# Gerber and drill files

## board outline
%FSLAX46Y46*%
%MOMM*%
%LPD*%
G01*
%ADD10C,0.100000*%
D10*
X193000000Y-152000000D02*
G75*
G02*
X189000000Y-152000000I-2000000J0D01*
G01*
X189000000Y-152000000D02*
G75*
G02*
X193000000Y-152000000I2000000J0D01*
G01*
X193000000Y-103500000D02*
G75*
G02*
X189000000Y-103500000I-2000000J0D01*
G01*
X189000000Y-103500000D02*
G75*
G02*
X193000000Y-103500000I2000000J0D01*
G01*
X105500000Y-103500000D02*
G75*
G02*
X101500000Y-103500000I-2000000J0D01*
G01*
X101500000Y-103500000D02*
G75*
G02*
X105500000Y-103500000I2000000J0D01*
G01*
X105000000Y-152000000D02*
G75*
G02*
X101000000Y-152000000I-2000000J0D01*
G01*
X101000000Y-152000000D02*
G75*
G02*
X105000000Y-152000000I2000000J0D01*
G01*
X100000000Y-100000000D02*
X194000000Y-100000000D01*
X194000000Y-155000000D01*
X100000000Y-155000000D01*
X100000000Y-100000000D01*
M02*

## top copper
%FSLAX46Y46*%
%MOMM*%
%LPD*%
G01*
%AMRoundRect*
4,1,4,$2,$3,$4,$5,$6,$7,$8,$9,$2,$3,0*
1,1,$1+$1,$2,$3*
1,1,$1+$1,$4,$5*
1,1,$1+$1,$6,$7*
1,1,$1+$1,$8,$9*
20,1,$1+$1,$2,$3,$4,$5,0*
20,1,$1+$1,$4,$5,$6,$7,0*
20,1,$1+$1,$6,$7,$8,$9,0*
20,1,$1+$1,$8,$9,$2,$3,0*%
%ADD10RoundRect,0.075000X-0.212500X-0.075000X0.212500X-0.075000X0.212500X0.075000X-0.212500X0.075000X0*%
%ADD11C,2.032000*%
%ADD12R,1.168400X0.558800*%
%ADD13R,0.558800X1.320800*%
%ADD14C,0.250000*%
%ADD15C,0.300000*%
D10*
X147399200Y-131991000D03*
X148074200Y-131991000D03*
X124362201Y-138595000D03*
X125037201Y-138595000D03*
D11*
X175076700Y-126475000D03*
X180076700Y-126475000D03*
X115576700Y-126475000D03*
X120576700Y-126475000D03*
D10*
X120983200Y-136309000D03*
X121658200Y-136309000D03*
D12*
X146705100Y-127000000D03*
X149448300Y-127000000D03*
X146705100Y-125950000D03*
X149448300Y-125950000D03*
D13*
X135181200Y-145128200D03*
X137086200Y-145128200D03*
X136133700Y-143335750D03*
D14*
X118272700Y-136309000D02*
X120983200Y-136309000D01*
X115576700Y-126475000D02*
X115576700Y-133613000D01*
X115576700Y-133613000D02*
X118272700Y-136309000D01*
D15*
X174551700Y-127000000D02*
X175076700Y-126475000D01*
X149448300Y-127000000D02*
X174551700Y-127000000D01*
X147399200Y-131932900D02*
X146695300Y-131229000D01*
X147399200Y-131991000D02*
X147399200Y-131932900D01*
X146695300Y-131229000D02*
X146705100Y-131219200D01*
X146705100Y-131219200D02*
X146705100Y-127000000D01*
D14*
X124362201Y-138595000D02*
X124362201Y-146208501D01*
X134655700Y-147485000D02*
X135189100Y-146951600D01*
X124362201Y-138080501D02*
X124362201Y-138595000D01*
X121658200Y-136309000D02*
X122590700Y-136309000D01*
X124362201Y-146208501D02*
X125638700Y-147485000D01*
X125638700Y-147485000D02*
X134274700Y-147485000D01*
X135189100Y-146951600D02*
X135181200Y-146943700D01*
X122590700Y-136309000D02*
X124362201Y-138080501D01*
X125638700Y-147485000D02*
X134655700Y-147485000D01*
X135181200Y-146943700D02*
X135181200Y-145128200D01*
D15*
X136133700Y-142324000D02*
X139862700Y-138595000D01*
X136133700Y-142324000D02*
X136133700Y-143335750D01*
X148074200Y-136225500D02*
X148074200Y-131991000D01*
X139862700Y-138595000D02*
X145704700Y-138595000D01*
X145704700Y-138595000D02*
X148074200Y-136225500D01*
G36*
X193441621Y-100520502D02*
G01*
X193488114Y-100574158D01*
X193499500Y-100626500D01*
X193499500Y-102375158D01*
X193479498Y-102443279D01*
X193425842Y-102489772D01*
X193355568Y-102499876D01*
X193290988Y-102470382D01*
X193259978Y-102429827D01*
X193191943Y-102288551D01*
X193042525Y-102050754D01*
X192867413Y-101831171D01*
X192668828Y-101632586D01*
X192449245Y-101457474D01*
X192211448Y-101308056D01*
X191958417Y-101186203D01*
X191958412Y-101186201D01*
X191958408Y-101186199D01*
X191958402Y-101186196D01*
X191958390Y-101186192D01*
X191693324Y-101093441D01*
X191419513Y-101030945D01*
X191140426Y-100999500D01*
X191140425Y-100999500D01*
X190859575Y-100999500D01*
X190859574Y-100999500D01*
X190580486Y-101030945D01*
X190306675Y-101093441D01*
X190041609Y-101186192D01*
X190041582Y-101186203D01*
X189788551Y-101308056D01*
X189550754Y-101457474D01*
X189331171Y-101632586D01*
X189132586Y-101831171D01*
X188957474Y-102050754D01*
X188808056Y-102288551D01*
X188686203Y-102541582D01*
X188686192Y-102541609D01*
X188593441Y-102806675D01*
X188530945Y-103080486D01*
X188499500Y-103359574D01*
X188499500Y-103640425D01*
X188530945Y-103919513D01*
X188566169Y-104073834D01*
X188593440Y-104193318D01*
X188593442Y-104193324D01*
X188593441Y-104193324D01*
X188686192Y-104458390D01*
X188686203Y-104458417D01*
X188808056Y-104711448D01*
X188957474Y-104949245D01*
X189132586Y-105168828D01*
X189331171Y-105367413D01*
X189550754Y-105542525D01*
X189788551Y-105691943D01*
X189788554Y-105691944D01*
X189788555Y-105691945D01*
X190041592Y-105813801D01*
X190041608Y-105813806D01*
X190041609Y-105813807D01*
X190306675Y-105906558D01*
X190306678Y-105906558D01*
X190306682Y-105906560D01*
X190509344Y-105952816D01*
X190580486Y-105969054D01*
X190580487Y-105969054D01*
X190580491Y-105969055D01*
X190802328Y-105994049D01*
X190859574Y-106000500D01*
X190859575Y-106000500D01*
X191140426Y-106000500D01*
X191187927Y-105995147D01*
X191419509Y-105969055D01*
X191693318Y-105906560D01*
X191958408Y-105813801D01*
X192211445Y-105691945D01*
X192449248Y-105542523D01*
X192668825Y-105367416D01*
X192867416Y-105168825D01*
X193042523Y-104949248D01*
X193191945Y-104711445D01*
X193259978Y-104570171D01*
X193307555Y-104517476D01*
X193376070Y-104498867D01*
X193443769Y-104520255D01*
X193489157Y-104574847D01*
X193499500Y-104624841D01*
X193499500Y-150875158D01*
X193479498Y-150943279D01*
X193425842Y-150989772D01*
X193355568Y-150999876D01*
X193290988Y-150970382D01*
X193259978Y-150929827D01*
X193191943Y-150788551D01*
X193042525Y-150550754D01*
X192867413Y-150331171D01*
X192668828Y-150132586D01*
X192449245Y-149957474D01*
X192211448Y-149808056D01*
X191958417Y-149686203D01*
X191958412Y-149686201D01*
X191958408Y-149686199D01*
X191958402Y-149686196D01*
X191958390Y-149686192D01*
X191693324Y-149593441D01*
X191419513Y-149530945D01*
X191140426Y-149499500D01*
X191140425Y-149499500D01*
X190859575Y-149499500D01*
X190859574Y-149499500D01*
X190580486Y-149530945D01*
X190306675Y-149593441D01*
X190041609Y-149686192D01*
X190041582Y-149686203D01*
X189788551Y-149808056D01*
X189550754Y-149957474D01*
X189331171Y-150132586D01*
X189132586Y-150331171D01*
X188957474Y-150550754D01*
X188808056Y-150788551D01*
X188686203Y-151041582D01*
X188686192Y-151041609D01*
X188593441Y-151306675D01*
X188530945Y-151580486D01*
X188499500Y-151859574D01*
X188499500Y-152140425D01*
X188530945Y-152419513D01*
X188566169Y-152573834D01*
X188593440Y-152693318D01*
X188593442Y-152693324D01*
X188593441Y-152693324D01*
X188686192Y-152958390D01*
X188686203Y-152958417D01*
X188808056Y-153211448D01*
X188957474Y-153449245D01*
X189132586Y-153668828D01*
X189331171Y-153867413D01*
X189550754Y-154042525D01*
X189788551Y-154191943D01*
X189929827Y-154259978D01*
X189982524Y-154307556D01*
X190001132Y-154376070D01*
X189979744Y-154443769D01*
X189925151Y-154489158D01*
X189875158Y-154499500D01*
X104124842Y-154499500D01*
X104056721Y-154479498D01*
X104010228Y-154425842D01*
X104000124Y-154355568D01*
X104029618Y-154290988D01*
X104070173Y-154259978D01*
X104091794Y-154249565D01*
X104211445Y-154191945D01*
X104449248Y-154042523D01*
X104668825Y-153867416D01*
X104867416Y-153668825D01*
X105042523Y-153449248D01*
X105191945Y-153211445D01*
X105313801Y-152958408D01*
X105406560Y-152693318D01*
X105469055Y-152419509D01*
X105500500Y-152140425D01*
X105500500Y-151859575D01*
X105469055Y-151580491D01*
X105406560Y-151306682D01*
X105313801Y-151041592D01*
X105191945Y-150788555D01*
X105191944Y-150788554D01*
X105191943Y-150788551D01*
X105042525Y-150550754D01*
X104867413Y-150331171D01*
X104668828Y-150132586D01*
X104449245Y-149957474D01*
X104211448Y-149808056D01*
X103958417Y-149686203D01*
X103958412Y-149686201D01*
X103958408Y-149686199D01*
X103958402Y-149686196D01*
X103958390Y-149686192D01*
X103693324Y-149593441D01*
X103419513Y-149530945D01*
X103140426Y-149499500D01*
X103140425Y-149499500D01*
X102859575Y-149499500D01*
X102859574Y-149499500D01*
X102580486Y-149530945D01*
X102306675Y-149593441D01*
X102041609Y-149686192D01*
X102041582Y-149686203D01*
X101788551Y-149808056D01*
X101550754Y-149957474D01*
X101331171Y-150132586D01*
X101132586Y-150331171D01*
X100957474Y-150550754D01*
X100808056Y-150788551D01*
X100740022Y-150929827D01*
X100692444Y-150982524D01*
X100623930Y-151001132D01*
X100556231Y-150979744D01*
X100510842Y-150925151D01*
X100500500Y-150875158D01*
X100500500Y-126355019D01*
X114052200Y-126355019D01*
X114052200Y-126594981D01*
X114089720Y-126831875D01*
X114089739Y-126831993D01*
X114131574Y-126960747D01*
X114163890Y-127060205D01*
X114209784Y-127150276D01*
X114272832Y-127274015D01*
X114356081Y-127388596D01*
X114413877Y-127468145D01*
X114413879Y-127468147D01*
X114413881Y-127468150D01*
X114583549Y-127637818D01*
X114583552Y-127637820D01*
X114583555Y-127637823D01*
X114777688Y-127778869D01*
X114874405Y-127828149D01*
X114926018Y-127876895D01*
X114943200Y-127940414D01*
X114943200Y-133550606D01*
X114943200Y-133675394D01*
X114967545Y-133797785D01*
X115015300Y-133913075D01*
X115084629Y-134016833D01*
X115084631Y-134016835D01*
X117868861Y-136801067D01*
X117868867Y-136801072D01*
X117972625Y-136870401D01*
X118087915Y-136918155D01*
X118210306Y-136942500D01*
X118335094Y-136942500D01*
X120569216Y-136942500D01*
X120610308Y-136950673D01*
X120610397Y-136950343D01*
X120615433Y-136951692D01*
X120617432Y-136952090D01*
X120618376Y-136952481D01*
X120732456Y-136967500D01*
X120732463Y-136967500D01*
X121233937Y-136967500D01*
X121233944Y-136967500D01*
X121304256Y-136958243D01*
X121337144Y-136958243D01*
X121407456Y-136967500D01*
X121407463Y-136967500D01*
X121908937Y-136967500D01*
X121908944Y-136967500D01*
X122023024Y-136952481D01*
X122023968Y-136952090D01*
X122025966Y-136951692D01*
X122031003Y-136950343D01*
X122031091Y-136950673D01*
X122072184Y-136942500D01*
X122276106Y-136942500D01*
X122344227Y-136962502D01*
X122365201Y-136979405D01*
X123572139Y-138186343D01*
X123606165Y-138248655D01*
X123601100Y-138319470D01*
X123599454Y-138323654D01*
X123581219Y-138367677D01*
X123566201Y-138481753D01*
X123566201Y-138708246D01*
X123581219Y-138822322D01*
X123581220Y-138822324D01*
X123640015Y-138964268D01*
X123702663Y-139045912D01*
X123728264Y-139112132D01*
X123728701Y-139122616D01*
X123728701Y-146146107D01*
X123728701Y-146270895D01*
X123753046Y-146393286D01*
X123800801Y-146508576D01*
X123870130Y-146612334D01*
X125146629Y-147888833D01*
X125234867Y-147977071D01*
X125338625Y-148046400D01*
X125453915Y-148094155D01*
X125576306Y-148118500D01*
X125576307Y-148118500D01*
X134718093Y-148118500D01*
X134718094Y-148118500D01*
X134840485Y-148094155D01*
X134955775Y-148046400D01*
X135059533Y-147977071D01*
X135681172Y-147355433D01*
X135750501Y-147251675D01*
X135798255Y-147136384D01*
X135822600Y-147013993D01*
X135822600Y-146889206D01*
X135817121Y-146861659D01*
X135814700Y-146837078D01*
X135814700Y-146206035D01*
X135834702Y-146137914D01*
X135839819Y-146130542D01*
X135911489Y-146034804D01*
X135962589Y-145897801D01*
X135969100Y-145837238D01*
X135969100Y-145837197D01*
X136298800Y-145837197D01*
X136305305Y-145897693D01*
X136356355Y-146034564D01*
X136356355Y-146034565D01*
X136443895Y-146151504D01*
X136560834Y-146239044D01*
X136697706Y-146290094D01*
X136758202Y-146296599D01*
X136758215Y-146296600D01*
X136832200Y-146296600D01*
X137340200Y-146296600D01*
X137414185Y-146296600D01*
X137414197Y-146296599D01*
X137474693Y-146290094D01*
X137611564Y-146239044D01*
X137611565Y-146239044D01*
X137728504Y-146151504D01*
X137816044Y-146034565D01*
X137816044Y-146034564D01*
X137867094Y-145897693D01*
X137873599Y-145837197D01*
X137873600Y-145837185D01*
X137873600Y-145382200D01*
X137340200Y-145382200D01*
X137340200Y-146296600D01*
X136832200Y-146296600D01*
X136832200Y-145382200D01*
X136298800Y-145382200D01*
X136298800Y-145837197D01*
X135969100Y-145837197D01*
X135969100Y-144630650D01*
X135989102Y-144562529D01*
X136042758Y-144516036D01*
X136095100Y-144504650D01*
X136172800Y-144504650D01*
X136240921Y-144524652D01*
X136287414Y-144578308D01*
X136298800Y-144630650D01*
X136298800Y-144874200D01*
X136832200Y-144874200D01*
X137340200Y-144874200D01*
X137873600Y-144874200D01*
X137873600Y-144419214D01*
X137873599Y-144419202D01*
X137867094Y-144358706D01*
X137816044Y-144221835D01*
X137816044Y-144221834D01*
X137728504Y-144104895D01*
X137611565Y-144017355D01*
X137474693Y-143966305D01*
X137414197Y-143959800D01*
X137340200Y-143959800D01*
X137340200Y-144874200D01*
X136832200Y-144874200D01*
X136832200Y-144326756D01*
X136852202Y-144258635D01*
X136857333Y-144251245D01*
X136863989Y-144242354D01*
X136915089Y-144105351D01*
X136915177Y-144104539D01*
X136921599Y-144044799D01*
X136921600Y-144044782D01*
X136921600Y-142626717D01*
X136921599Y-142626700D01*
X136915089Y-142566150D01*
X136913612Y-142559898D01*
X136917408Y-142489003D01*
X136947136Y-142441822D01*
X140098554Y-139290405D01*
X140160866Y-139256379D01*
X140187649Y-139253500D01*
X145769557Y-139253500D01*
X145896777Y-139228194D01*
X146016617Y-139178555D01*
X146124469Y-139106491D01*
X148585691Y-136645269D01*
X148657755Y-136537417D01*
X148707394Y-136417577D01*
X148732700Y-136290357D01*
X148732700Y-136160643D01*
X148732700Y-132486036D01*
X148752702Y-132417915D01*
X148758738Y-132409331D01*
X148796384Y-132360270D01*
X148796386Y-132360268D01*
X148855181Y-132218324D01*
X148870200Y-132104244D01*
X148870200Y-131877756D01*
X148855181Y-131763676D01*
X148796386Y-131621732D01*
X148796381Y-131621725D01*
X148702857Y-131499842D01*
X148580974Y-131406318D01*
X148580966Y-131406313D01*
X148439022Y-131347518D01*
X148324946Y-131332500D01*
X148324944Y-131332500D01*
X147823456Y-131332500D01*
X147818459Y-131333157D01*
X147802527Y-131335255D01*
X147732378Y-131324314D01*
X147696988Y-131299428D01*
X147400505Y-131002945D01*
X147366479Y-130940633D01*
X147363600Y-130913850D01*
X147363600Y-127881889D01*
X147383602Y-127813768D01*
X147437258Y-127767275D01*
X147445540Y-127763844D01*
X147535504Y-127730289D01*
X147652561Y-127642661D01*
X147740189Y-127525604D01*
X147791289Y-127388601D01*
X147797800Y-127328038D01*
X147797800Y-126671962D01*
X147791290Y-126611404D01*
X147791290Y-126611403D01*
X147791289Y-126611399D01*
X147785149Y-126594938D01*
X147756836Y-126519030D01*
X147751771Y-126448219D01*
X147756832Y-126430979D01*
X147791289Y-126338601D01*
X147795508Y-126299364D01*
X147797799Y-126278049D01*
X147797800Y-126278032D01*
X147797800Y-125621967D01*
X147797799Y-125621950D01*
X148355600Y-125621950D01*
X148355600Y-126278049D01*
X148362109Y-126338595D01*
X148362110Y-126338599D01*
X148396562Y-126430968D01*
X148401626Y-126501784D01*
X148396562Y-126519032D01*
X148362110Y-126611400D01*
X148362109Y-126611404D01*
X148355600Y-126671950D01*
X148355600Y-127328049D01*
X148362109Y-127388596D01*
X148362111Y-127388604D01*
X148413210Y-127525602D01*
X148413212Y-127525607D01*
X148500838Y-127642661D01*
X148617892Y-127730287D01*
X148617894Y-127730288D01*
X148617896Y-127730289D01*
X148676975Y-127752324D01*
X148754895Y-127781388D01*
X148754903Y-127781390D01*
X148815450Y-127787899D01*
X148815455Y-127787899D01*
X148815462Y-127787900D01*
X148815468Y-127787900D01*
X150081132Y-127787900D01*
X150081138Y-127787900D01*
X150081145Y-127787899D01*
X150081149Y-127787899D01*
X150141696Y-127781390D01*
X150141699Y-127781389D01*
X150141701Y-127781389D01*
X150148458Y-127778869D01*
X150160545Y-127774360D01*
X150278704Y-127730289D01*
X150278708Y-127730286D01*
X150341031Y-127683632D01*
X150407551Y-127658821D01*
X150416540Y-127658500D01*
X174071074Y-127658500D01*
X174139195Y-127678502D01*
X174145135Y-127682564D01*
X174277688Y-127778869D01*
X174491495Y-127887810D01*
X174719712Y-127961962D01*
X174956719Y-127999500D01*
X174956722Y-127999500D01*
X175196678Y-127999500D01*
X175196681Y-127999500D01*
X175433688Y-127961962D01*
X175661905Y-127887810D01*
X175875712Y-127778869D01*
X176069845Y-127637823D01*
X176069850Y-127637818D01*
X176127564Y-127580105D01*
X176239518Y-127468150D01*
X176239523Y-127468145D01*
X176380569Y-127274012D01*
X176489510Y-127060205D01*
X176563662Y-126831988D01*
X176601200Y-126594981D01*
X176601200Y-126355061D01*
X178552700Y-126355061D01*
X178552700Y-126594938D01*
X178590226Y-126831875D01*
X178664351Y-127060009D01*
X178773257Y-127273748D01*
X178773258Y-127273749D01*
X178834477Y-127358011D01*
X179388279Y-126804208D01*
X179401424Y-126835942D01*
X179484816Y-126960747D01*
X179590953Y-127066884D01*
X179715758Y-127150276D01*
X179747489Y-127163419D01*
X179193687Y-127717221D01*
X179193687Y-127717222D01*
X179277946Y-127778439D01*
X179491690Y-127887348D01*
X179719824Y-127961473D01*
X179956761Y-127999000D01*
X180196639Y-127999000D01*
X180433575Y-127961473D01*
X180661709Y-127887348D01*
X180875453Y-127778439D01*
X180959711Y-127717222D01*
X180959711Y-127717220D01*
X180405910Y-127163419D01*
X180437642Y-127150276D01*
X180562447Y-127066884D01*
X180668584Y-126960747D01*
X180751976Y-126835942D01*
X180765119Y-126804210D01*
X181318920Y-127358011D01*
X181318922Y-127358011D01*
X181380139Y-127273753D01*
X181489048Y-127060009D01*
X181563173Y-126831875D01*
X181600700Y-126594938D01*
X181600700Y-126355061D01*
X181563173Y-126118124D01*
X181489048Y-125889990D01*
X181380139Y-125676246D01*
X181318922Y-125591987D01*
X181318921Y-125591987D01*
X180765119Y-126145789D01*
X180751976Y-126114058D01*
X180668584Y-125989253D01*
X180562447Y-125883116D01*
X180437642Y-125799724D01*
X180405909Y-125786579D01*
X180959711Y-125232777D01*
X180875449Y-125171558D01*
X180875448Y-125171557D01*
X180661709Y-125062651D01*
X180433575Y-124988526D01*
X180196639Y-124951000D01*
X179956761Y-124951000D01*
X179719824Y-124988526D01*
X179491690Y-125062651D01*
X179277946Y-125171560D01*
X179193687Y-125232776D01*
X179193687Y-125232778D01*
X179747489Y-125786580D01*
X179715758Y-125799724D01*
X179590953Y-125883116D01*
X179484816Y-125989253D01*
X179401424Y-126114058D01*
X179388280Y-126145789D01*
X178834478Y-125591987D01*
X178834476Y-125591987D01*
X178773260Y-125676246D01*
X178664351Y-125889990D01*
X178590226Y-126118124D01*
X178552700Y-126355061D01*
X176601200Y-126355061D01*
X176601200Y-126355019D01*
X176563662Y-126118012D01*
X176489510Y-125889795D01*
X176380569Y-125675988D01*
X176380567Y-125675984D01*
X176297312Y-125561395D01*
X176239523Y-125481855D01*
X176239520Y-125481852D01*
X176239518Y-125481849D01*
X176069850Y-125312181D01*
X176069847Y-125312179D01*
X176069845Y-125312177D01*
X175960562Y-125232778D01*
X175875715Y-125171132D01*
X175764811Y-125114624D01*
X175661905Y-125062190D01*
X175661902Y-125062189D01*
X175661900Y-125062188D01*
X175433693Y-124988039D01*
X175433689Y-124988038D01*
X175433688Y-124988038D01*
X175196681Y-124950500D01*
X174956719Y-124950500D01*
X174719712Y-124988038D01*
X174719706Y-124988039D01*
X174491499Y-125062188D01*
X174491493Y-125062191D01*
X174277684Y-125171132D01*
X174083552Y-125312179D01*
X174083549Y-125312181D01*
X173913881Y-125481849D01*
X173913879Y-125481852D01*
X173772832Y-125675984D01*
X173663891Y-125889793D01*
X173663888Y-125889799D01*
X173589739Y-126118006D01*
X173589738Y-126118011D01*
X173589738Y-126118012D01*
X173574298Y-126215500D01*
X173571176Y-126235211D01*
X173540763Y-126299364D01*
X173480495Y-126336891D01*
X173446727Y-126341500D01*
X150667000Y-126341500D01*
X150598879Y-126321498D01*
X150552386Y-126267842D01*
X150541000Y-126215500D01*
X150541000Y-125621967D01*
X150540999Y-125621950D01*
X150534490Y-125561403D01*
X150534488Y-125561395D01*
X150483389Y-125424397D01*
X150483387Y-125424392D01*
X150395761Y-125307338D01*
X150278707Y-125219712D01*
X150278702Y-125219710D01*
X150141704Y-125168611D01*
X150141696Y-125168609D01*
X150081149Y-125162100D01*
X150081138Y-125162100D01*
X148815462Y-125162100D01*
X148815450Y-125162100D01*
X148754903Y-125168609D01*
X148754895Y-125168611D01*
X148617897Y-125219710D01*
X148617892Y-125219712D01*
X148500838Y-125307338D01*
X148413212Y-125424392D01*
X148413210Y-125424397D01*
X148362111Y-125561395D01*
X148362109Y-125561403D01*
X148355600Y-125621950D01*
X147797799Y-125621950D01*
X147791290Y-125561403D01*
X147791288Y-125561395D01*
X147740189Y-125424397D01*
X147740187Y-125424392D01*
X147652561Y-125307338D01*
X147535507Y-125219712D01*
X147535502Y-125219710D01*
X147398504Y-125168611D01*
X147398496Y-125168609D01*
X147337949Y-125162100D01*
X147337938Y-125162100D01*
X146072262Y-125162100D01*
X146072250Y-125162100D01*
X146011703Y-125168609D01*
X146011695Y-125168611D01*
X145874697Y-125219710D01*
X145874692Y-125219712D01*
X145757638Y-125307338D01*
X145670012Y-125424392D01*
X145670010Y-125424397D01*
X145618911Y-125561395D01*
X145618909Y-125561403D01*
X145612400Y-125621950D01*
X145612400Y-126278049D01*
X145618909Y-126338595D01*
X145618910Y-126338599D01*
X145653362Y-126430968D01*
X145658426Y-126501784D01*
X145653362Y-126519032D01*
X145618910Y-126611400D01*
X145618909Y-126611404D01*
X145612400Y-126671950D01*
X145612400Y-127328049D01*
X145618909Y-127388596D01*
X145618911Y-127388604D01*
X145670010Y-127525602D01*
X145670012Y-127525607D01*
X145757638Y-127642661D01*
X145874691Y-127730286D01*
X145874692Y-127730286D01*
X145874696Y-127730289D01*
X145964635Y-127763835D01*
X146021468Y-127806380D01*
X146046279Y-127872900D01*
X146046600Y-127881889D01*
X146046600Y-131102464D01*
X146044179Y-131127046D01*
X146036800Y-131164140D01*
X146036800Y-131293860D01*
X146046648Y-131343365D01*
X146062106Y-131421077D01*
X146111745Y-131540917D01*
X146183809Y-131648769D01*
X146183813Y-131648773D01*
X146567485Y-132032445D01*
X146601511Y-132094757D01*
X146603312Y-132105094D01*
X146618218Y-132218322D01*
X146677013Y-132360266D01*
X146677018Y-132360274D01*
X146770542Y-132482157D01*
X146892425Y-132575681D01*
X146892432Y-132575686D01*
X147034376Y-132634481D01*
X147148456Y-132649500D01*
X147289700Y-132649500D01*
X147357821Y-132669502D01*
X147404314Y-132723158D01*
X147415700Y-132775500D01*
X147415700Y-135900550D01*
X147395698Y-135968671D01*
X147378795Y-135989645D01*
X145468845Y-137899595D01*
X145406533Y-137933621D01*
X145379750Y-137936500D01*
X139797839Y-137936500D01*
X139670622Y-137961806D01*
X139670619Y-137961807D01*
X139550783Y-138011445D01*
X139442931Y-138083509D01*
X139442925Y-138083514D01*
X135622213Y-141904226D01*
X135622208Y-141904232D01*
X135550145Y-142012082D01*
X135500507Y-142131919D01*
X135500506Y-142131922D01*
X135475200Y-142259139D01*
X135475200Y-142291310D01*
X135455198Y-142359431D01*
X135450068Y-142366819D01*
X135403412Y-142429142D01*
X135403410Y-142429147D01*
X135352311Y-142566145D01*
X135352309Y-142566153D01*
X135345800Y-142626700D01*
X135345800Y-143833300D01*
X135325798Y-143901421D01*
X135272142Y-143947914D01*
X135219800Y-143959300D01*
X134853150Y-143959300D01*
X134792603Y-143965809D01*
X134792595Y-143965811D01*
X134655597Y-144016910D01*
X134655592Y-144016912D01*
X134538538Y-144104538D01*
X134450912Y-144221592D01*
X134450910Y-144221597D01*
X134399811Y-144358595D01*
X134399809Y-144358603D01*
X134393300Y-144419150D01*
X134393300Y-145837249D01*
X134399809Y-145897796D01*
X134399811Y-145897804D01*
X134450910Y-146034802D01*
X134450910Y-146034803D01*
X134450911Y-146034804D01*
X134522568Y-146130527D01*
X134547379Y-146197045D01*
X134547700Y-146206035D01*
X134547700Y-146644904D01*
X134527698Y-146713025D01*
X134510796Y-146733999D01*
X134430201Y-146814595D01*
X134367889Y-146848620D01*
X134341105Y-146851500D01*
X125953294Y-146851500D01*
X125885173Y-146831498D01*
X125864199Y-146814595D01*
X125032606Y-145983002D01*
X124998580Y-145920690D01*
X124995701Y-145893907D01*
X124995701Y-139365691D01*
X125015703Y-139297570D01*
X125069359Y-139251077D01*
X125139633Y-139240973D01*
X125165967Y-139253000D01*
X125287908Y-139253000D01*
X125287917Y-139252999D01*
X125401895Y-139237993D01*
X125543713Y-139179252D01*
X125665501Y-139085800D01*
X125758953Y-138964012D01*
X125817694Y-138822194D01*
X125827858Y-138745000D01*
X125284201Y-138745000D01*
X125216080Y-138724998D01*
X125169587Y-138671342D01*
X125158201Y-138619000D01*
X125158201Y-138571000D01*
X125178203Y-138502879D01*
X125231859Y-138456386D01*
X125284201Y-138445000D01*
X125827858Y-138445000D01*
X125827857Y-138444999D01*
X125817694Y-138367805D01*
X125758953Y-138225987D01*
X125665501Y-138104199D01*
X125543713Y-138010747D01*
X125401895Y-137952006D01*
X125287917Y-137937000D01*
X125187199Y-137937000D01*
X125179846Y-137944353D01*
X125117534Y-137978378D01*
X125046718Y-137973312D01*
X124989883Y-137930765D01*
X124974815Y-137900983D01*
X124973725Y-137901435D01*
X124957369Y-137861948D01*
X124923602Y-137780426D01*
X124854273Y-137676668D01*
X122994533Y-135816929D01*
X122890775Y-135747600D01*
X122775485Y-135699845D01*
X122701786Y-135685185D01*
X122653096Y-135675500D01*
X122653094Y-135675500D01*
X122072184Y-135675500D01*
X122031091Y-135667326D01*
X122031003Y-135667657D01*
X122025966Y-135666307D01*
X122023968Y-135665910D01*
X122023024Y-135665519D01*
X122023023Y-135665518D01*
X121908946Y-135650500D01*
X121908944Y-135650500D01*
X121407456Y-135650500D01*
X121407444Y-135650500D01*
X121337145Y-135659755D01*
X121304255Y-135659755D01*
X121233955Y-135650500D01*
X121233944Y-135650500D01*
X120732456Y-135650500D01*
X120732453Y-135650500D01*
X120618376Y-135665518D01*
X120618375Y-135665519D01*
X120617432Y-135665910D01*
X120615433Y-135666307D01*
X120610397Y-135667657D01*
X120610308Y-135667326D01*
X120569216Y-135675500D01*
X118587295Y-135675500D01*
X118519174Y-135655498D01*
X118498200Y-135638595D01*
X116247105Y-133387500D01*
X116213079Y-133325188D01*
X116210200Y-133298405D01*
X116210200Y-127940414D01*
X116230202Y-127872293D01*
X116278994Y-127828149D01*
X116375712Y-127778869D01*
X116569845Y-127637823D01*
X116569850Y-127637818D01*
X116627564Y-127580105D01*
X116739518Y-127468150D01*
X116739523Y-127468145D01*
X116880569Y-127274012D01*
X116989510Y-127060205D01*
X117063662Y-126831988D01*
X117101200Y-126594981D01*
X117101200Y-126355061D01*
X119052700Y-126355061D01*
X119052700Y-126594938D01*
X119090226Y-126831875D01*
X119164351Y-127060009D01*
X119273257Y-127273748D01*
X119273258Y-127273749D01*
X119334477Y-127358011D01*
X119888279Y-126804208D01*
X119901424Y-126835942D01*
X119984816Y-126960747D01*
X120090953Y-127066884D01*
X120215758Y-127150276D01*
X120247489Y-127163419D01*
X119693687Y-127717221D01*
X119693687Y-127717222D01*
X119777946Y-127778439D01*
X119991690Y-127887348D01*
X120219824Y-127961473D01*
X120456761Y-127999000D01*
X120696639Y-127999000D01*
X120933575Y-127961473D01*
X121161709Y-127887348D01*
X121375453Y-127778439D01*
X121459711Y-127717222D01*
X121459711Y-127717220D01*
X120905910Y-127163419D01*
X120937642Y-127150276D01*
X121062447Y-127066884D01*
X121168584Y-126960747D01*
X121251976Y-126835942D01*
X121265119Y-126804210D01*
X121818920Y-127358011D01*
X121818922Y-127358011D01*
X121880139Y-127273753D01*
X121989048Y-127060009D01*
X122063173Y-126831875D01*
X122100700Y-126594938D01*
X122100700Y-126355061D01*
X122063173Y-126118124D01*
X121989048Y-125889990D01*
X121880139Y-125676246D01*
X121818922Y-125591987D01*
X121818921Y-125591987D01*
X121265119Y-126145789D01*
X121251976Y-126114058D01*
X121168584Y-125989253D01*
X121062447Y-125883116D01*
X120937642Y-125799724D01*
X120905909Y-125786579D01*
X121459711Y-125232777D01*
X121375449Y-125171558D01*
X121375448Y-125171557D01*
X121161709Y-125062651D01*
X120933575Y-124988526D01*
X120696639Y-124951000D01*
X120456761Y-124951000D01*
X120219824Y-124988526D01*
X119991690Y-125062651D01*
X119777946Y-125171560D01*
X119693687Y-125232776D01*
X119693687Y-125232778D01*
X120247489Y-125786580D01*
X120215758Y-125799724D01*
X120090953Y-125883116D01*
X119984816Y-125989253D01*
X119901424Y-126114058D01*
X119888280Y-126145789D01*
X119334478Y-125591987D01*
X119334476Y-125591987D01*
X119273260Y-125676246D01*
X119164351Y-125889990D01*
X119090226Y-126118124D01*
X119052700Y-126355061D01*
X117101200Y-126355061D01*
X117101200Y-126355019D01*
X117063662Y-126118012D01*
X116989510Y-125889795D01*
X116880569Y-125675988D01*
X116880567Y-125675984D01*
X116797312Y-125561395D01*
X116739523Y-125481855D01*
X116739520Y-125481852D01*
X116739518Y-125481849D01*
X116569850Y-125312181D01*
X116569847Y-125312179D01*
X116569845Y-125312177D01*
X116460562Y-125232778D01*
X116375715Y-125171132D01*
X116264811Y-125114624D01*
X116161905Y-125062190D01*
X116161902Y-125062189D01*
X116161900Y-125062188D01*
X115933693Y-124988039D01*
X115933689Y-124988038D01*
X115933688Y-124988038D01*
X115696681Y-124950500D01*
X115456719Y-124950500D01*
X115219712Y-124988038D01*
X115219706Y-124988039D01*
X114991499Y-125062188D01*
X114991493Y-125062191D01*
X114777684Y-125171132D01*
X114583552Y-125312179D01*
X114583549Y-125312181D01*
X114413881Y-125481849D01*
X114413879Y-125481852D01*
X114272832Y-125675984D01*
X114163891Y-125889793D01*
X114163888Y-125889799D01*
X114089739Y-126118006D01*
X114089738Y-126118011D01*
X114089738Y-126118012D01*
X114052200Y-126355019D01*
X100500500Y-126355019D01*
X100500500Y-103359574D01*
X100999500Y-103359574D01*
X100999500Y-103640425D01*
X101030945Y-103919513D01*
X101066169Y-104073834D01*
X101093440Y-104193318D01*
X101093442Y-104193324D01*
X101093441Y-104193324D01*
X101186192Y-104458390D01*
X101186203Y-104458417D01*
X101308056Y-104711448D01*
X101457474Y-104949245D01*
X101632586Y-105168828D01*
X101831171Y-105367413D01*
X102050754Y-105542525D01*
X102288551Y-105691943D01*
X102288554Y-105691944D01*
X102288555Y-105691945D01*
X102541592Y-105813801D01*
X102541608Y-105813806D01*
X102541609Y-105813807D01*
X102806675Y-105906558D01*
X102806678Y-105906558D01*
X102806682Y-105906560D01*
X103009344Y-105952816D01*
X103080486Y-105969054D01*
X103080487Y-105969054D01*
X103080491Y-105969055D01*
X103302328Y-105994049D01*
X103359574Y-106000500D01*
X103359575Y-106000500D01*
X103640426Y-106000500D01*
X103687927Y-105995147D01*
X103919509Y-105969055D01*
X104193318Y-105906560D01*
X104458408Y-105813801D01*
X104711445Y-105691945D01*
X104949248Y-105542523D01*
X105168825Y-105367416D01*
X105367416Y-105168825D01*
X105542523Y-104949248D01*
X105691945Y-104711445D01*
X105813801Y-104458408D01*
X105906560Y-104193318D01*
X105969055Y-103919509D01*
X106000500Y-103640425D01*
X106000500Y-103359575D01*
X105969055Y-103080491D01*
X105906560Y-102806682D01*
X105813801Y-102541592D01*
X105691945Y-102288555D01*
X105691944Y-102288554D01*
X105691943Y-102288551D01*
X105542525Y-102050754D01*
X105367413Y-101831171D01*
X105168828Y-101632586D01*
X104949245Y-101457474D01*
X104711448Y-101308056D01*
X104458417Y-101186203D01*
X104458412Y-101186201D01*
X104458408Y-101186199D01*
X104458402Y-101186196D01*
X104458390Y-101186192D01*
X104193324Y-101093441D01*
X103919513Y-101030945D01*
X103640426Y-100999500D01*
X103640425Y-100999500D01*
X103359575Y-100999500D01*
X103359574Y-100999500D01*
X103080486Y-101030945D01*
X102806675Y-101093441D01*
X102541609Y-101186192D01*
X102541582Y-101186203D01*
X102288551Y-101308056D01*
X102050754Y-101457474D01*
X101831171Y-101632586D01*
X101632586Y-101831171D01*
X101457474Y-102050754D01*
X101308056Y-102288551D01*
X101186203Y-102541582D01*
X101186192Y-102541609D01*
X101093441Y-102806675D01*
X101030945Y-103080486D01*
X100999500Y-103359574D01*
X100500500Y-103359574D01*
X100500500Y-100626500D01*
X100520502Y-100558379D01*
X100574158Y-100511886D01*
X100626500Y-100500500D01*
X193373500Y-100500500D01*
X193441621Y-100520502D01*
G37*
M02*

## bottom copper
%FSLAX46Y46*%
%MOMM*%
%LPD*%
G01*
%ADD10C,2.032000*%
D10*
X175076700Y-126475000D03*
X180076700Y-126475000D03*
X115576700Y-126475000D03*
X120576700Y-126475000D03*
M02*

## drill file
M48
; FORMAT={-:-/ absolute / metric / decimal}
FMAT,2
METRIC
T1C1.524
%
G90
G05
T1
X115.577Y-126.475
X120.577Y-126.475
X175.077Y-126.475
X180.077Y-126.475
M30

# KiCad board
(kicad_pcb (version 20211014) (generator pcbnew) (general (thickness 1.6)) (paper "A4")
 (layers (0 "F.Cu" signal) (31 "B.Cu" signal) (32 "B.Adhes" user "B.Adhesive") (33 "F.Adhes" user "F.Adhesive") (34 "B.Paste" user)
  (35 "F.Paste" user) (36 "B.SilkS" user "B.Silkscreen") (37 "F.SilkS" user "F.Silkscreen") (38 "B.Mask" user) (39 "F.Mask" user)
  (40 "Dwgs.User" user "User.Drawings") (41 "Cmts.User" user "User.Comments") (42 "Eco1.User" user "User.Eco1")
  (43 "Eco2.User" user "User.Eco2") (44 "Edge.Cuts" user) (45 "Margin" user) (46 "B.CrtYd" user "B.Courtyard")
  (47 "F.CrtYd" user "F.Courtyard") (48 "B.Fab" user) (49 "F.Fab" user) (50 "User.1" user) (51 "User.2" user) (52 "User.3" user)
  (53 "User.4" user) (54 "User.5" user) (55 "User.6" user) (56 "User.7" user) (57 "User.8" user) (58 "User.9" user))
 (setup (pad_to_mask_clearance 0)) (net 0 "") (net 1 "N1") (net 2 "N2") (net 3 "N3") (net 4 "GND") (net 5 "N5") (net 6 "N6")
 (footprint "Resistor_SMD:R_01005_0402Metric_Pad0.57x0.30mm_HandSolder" (layer "F.Cu") (at 147.7367 131.991)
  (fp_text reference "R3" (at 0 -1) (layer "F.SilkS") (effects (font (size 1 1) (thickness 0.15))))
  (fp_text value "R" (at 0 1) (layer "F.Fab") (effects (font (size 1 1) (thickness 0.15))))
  (pad "" smd roundrect (at -0.3625 0) (size 0.41 0.27) (layers "F.Paste") (roundrect_rratio 0.25))
  (pad "" smd roundrect (at 0.3625 0) (size 0.41 0.27) (layers "F.Paste") (roundrect_rratio 0.25))
  (pad "1" smd roundrect (at -0.3375 0) (size 0.575 0.3) (layers "F.Cu" "F.Mask") (roundrect_rratio 0.25) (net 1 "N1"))
  (pad "2" smd roundrect (at 0.3375 0) (size 0.575 0.3) (layers "F.Cu" "F.Mask") (roundrect_rratio 0.25) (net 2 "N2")))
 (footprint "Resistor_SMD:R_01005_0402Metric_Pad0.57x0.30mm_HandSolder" (layer "F.Cu") (at 124.699701 138.595)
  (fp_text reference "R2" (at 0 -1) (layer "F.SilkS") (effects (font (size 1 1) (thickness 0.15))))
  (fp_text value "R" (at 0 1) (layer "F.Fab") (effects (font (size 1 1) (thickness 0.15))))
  (pad "" smd roundrect (at -0.3625 0) (size 0.41 0.27) (layers "F.Paste") (roundrect_rratio 0.25))
  (pad "" smd roundrect (at 0.3625 0) (size 0.41 0.27) (layers "F.Paste") (roundrect_rratio 0.25))
  (pad "1" smd roundrect (at -0.3375 0) (size 0.575 0.3) (layers "F.Cu" "F.Mask") (roundrect_rratio 0.25) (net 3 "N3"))
  (pad "2" smd roundrect (at 0.3375 0) (size 0.575 0.3) (layers "F.Cu" "F.Mask") (roundrect_rratio 0.25) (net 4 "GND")))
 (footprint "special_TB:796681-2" (layer "F.Cu") (at 175.0767 126.475)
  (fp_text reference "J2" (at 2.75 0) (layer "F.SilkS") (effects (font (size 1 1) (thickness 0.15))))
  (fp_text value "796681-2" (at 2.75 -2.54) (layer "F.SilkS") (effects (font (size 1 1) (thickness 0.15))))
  (pad "1" thru_hole circle (at 0 0) (size 2.032 2.032) (drill 1.524) (layers *.Cu *.Mask) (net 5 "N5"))
  (pad "2" thru_hole circle (at 5 0) (size 2.032 2.032) (drill 1.524) (layers *.Cu *.Mask) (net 4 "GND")))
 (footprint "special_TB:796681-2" (layer "F.Cu") (at 115.5767 126.475)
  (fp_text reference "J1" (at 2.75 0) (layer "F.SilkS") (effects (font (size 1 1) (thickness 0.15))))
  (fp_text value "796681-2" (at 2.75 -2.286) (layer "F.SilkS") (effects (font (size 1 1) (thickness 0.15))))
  (pad "1" thru_hole circle (at 0 0) (size 2.032 2.032) (drill 1.524) (layers *.Cu *.Mask) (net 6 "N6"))
  (pad "2" thru_hole circle (at 5 0) (size 2.032 2.032) (drill 1.524) (layers *.Cu *.Mask) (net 4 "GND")))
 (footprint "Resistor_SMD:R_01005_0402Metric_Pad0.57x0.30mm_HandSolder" (layer "F.Cu") (at 121.3207 136.309)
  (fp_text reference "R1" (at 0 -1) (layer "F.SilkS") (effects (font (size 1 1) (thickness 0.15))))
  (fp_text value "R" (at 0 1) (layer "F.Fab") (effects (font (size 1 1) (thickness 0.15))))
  (pad "" smd roundrect (at 0.3625 0) (size 0.41 0.27) (layers "F.Paste") (roundrect_rratio 0.25))
  (pad "" smd roundrect (at -0.3625 0) (size 0.41 0.27) (layers "F.Paste") (roundrect_rratio 0.25))
  (pad "1" smd roundrect (at -0.3375 0) (size 0.575 0.3) (layers "F.Cu" "F.Mask") (roundrect_rratio 0.25) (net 6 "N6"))
  (pad "2" smd roundrect (at 0.3375 0) (size 0.575 0.3) (layers "F.Cu" "F.Mask") (roundrect_rratio 0.25) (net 3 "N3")))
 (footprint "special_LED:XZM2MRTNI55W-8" (layer "F.Cu") (at 148.0767 126.475)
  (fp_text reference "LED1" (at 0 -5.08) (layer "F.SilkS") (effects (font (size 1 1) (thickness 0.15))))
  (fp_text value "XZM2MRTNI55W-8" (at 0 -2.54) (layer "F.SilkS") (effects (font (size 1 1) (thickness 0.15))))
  (pad "1" smd rect (at -1.3716 0.525) (size 1.1684 0.5588) (layers "F.Cu" "F.Paste" "F.Mask") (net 1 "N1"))
  (pad "2" smd rect (at 1.3716 0.525) (size 1.1684 0.5588) (layers "F.Cu" "F.Paste" "F.Mask") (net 5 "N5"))
  (pad "3" smd rect (at -1.3716 -0.525) (size 1.1684 0.5588) (layers "F.Cu" "F.Paste" "F.Mask"))
  (pad "4" smd rect (at 1.3716 -0.525) (size 1.1684 0.5588) (layers "F.Cu" "F.Paste" "F.Mask")))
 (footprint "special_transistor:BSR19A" (layer "F.Cu") (at 136.1337 144.183)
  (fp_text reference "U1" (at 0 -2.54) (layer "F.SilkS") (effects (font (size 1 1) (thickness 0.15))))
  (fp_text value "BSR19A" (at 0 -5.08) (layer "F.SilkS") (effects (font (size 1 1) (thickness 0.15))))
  (pad "1" smd rect (at -0.9525 0.9452) (size 0.5588 1.3208) (layers "F.Cu" "F.Paste" "F.Mask") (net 3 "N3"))
  (pad "2" smd rect (at 0.9525 0.9452) (size 0.5588 1.3208) (layers "F.Cu" "F.Paste" "F.Mask") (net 4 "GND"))
  (pad "3" smd rect (at 0 -0.84725) (size 0.5588 1.3208) (layers "F.Cu" "F.Paste" "F.Mask") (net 2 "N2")))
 (gr_circle (center 191 152) (end 193 152) (layer "Edge.Cuts") (width 0.1) (fill none))
 (gr_circle (center 191 103.5) (end 193 103.5) (layer "Edge.Cuts") (width 0.1) (fill none))
 (gr_circle (center 103.5 103.5) (end 105.5 103.5) (layer "Edge.Cuts") (width 0.1) (fill none))
 (gr_circle (center 103 152) (end 105 152) (layer "Edge.Cuts") (width 0.1) (fill none))
 (gr_rect (start 100 100) (end 194 155) (layer "Edge.Cuts") (width 0.1) (fill none))
 (segment (start 118.2727 136.309) (end 120.9832 136.309) (width 0.25) (layer "F.Cu") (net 6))
 (segment (start 115.5767 126.475) (end 115.5767 133.613) (width 0.25) (layer "F.Cu") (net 6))
 (segment (start 115.5767 133.613) (end 118.2727 136.309) (width 0.25) (layer "F.Cu") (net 6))
 (segment (start 174.5517 127) (end 175.0767 126.475) (width 0.3) (layer "F.Cu") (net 5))
 (segment (start 149.4483 127) (end 174.5517 127) (width 0.3) (layer "F.Cu") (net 5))
 (segment (start 147.3992 131.9329) (end 146.6953 131.229) (width 0.3) (layer "F.Cu") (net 1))
 (segment (start 147.3992 131.991) (end 147.3992 131.9329) (width 0.3) (layer "F.Cu") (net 1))
 (segment (start 146.6953 131.229) (end 146.7051 131.2192) (width 0.3) (layer "F.Cu") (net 1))
 (segment (start 146.7051 131.2192) (end 146.7051 127) (width 0.3) (layer "F.Cu") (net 1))
 (segment (start 124.362201 138.595) (end 124.362201 146.208501) (width 0.25) (layer "F.Cu") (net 3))
 (segment (start 134.6557 147.485) (end 135.1891 146.9516) (width 0.25) (layer "F.Cu") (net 3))
 (segment (start 124.362201 138.080501) (end 124.362201 138.595) (width 0.25) (layer "F.Cu") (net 3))
 (segment (start 121.6582 136.309) (end 122.5907 136.309) (width 0.25) (layer "F.Cu") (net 3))
 (segment (start 124.362201 146.208501) (end 125.6387 147.485) (width 0.25) (layer "F.Cu") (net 3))
 (segment (start 125.6387 147.485) (end 134.2747 147.485) (width 0.25) (layer "F.Cu") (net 3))
 (segment (start 135.1891 146.9516) (end 135.1812 146.9437) (width 0.25) (layer "F.Cu") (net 3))
 (segment (start 122.5907 136.309) (end 124.362201 138.080501) (width 0.25) (layer "F.Cu") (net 3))
 (segment (start 125.6387 147.485) (end 134.6557 147.485) (width 0.25) (layer "F.Cu") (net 3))
 (segment (start 135.1812 146.9437) (end 135.1812 145.1282) (width 0.25) (layer "F.Cu") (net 3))
 (segment (start 136.1337 142.324) (end 139.8627 138.595) (width 0.3) (layer "F.Cu") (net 2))
 (segment (start 136.1337 142.324) (end 136.1337 143.33575) (width 0.3) (layer "F.Cu") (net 2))
 (segment (start 148.0742 136.2255) (end 148.0742 131.991) (width 0.3) (layer "F.Cu") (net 2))
 (segment (start 139.8627 138.595) (end 145.7047 138.595) (width 0.3) (layer "F.Cu") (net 2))
 (segment (start 145.7047 138.595) (end 148.0742 136.2255) (width 0.3) (layer "F.Cu") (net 2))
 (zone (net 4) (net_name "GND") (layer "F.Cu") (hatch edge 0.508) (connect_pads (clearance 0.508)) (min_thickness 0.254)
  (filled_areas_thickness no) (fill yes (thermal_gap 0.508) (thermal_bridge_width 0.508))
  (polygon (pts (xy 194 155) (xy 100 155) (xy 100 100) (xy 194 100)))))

